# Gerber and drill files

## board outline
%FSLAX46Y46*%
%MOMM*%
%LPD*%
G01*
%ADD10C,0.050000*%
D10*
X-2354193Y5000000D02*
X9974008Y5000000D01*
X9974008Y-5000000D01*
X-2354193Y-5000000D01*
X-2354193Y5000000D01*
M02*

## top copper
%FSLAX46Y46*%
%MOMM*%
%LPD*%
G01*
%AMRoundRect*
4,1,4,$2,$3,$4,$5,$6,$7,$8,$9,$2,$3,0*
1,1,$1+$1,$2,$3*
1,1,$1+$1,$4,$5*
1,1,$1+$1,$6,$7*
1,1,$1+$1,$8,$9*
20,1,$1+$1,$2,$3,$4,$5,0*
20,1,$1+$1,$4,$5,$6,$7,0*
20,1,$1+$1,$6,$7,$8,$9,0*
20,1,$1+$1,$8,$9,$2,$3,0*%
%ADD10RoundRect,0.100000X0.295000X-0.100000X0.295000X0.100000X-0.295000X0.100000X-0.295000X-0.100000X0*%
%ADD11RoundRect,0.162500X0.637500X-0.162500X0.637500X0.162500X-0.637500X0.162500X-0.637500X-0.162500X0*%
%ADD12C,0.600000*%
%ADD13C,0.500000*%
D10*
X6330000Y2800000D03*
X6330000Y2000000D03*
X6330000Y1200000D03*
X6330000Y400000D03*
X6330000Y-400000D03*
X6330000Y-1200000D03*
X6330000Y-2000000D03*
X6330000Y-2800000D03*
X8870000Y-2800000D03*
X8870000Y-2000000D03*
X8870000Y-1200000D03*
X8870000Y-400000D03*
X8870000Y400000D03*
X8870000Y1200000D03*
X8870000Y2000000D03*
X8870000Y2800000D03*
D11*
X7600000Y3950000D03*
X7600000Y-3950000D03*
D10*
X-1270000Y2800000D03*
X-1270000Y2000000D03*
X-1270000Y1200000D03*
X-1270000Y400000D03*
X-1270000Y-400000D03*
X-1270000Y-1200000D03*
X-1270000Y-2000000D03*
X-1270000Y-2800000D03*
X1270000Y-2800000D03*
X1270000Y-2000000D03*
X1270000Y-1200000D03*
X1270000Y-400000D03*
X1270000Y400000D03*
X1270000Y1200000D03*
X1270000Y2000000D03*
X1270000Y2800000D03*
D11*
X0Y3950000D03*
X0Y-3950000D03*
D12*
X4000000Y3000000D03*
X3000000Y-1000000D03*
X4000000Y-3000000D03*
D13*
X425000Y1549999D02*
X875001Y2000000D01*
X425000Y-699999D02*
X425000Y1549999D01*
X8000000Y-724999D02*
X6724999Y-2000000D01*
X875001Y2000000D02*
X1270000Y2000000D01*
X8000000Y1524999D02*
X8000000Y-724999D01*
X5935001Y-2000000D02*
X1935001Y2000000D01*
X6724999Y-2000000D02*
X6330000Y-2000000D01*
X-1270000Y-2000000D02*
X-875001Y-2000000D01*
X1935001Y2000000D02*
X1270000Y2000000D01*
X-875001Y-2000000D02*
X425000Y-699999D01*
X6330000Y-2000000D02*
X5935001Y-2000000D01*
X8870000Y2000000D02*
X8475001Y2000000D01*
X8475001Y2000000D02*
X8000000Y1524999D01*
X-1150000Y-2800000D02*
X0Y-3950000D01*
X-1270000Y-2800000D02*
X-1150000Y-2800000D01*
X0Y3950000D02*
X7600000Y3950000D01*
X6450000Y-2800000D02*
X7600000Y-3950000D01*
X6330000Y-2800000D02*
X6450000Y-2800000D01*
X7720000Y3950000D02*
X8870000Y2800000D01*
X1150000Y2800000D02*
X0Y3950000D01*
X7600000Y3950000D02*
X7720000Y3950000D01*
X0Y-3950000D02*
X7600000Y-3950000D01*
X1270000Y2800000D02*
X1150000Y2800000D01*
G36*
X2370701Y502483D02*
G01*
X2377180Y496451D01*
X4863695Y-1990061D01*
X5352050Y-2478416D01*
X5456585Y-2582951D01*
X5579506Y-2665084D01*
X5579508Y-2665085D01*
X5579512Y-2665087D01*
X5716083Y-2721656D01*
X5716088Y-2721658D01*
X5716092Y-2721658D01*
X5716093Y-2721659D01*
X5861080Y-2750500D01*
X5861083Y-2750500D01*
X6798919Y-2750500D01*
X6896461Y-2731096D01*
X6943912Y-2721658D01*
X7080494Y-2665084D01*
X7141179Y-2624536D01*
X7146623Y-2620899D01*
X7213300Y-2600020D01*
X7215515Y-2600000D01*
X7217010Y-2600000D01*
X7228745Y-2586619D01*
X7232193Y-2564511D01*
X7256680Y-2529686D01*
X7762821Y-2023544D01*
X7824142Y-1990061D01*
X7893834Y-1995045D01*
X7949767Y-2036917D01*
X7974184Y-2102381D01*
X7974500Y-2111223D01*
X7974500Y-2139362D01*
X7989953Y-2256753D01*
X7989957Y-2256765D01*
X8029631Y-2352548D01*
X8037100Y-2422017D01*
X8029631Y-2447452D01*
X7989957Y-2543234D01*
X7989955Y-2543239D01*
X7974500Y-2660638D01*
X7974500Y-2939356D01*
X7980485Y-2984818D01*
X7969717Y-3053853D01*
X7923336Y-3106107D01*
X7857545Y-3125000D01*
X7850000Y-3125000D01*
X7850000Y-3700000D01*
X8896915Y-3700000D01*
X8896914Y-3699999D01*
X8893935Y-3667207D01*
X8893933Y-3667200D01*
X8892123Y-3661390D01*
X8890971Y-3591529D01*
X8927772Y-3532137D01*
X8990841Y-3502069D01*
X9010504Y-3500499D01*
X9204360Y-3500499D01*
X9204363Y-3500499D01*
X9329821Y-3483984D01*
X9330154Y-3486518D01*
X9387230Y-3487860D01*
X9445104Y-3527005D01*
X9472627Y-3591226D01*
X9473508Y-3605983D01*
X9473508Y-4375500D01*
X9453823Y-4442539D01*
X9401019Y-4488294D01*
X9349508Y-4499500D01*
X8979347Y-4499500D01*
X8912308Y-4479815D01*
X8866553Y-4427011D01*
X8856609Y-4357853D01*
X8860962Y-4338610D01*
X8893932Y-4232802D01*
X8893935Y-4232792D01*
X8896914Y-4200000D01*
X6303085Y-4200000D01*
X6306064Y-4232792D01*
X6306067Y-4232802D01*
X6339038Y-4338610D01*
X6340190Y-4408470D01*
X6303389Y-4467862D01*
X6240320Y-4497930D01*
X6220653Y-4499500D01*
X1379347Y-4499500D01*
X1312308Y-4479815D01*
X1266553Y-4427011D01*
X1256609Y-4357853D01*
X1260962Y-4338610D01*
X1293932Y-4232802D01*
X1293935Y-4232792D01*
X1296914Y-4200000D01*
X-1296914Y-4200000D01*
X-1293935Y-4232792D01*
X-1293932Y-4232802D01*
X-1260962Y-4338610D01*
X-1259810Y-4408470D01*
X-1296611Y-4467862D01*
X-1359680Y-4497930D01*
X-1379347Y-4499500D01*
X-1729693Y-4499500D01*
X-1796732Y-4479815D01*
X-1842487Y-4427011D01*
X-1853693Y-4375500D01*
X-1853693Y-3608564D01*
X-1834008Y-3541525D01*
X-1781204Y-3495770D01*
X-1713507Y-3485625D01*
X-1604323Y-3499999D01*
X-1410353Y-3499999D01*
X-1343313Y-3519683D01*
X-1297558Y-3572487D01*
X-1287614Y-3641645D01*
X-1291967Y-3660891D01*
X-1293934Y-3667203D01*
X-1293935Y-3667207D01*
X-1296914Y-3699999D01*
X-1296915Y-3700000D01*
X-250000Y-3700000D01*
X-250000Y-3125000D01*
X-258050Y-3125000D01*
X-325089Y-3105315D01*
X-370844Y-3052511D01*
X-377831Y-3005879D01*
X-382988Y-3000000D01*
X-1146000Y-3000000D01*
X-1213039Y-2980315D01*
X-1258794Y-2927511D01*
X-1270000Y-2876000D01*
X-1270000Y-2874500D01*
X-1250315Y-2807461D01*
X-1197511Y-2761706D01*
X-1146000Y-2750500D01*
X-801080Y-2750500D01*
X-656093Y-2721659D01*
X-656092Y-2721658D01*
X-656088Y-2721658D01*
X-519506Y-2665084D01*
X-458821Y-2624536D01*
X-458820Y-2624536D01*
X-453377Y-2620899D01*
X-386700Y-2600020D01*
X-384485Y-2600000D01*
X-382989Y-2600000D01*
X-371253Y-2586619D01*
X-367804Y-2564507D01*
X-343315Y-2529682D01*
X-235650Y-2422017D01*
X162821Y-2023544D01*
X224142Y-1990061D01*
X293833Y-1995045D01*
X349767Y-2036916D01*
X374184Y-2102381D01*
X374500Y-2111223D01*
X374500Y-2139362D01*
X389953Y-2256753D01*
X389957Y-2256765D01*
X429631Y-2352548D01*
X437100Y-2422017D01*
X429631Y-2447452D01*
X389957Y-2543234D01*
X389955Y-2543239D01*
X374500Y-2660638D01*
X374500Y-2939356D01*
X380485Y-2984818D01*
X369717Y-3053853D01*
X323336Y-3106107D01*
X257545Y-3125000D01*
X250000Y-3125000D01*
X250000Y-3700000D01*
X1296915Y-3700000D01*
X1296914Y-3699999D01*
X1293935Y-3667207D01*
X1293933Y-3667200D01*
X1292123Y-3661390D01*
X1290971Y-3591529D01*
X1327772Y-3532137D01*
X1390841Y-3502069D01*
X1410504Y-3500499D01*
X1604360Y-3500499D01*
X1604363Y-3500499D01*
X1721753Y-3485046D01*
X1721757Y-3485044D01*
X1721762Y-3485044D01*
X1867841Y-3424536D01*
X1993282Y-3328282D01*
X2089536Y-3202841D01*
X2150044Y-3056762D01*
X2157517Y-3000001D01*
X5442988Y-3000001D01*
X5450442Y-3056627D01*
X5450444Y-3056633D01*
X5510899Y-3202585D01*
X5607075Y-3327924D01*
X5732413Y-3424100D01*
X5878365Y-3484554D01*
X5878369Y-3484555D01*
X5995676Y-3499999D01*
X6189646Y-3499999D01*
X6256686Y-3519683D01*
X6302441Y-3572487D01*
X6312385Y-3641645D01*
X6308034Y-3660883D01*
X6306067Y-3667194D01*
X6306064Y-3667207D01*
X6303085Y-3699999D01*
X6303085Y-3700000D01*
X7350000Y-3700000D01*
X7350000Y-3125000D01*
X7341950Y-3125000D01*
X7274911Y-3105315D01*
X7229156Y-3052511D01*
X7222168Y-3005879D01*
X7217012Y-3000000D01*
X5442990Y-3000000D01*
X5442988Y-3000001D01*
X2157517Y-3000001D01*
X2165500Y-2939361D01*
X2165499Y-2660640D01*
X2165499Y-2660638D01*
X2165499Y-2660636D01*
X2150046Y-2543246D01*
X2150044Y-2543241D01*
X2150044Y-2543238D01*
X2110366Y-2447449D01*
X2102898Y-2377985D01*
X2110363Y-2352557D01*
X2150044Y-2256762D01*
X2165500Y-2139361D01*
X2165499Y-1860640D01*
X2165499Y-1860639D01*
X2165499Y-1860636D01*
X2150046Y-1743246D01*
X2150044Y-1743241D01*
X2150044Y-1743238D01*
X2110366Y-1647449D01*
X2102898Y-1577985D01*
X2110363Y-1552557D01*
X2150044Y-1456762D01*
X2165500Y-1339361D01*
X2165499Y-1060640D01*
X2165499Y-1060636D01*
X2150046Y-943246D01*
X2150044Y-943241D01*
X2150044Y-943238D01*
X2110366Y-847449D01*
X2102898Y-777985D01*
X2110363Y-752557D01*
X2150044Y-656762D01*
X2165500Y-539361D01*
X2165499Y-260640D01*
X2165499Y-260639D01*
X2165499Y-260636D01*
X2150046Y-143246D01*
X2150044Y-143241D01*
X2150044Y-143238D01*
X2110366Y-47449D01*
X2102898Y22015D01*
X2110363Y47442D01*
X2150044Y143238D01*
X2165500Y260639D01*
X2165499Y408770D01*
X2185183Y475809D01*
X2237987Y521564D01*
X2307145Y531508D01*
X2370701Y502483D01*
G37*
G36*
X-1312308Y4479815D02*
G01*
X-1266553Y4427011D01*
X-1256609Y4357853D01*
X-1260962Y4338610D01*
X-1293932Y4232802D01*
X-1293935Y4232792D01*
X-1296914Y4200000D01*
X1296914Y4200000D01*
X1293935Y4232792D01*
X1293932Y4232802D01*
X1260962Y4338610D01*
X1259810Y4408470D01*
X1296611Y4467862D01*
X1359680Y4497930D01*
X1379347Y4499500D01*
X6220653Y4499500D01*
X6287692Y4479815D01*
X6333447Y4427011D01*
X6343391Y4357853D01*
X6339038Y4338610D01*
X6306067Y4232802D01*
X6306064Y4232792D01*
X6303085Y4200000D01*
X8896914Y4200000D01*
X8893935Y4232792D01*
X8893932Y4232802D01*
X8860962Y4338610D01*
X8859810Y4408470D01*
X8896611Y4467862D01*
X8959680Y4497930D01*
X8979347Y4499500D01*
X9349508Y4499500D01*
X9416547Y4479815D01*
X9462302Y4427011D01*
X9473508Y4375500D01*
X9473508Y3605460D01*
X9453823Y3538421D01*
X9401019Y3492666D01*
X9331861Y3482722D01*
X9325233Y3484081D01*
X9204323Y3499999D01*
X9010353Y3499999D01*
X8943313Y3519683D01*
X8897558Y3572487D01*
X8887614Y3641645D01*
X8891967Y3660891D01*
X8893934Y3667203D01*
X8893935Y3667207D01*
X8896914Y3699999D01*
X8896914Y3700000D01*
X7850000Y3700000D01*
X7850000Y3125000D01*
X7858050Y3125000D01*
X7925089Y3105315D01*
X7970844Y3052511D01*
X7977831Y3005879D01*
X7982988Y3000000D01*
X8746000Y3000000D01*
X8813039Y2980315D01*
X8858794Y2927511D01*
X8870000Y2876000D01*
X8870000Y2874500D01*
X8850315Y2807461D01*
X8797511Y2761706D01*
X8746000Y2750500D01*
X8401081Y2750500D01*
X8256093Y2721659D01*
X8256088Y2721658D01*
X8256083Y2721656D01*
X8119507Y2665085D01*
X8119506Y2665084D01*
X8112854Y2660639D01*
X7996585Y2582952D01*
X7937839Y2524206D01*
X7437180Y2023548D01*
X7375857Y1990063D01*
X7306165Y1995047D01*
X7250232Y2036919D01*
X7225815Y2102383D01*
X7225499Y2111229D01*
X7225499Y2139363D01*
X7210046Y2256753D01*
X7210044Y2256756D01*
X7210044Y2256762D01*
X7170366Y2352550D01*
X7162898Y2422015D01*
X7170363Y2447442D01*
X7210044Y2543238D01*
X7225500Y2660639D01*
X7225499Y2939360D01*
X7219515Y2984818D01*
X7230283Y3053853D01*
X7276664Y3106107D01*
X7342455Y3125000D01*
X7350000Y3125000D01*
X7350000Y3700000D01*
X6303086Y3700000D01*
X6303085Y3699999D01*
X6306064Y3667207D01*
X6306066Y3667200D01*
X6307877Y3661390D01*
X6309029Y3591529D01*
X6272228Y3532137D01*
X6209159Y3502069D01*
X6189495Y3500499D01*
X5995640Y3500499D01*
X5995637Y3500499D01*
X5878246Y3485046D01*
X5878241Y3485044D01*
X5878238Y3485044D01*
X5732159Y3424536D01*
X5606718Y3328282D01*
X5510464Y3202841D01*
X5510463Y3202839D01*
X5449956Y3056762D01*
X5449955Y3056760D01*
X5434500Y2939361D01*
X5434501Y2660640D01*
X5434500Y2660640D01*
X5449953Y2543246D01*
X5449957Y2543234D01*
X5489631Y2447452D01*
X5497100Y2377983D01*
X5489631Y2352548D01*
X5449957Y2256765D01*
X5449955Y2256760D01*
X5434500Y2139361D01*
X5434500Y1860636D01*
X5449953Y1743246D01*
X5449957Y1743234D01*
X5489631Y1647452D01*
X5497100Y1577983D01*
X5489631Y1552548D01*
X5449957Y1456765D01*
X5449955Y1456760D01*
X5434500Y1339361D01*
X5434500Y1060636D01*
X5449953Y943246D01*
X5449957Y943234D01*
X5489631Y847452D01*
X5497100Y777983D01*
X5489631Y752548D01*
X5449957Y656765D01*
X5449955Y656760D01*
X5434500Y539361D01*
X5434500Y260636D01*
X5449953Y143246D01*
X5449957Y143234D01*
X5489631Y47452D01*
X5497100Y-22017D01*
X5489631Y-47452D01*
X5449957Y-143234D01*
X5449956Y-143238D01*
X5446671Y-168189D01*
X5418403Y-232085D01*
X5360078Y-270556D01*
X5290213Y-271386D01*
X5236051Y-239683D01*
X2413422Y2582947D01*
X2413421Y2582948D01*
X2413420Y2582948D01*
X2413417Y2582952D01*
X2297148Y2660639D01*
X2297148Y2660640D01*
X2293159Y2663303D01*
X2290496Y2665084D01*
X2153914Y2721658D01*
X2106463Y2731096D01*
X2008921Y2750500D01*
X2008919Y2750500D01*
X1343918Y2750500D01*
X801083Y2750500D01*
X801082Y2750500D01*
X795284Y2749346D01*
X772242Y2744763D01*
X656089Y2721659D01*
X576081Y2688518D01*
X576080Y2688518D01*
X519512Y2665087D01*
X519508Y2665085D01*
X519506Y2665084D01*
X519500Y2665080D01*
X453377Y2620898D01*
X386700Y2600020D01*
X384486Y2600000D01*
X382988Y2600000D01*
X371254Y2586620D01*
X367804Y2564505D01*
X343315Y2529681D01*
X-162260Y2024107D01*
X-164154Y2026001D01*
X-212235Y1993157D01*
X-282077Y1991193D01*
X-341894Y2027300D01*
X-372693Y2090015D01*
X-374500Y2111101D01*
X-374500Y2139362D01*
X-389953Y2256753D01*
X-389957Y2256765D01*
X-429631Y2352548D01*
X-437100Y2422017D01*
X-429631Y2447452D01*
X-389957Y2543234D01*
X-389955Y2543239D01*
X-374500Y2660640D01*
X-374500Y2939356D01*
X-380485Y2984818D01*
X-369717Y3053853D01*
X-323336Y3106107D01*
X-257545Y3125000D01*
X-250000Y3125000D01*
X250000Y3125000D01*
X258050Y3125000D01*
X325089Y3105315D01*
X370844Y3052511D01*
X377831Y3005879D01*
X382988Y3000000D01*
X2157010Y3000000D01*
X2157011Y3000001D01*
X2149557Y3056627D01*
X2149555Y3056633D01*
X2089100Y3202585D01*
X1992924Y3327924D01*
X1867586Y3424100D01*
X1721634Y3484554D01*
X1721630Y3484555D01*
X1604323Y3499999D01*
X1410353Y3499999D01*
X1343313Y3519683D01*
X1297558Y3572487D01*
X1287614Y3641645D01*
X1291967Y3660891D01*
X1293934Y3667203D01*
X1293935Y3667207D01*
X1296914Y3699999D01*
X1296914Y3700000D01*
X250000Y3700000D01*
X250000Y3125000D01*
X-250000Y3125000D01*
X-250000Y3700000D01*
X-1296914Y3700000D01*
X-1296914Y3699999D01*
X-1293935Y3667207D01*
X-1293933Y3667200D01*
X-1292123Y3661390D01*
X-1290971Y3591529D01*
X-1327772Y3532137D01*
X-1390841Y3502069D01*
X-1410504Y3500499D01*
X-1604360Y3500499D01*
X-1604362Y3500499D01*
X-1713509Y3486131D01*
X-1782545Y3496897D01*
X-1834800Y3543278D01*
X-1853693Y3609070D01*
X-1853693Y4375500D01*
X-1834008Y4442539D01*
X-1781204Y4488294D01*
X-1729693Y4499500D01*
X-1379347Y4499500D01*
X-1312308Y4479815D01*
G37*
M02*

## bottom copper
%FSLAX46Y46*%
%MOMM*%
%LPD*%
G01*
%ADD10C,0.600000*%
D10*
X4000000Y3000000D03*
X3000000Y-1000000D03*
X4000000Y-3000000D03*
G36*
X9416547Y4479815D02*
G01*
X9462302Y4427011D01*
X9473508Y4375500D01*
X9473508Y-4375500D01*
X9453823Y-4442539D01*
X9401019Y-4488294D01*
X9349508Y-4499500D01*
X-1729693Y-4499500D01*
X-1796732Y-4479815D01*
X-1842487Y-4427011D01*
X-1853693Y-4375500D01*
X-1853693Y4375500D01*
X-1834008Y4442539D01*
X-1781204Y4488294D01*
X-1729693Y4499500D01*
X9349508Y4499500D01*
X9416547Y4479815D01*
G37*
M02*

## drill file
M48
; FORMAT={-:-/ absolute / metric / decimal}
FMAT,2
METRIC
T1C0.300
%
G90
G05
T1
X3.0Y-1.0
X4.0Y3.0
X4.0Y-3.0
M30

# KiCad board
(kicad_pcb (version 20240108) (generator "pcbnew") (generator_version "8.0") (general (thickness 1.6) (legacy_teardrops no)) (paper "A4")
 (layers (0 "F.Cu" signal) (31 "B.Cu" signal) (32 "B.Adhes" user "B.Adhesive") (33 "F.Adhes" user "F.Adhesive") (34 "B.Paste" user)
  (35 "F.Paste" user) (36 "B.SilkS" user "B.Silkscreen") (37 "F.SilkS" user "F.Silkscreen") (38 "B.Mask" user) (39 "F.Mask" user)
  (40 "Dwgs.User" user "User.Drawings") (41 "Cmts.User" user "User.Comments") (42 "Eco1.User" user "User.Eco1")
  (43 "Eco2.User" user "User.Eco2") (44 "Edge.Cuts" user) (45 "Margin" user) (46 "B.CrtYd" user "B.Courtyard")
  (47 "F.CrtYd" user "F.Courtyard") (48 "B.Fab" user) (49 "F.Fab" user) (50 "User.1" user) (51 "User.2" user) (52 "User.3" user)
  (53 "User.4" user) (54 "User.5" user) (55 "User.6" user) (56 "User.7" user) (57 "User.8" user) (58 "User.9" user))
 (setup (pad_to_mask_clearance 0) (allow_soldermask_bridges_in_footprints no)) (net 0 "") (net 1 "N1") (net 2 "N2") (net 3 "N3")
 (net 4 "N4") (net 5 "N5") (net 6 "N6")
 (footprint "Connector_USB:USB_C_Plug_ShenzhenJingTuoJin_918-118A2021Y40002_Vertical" (layer "F.Cu") (at 7.6 0)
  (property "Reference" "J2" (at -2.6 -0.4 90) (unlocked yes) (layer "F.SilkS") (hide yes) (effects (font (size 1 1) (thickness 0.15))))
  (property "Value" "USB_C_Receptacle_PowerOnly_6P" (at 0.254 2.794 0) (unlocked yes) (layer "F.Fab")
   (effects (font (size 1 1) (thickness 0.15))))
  (pad "A1" smd roundrect (at -1.27 -2.8 90) (size 0.4 0.79) (layers "F.Cu" "F.Paste" "F.Mask") (roundrect_rratio 0.25))
  (pad "A4" smd roundrect (at -1.27 -2 90) (size 0.4 0.79) (layers "F.Cu" "F.Paste" "F.Mask") (roundrect_rratio 0.25))
  (pad "A5" smd roundrect (at -1.27 -1.2 90) (size 0.4 0.79) (layers "F.Cu" "F.Paste" "F.Mask") (roundrect_rratio 0.25) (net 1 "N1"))
  (pad "A6" smd roundrect (at -1.27 -0.4 90) (size 0.4 0.79) (layers "F.Cu" "F.Paste" "F.Mask") (roundrect_rratio 0.25))
  (pad "A7" smd roundrect (at -1.27 0.4 90) (size 0.4 0.79) (layers "F.Cu" "F.Paste" "F.Mask") (roundrect_rratio 0.25))
  (pad "A8" smd roundrect (at -1.27 1.2 90) (size 0.4 0.79) (layers "F.Cu" "F.Paste" "F.Mask") (roundrect_rratio 0.25))
  (pad "A9" smd roundrect (at -1.27 2 90) (size 0.4 0.79) (layers "F.Cu" "F.Paste" "F.Mask") (roundrect_rratio 0.25) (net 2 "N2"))
  (pad "A12" smd roundrect (at -1.27 2.8 90) (size 0.4 0.79) (layers "F.Cu" "F.Paste" "F.Mask") (roundrect_rratio 0.25) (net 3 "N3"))
  (pad "B1" smd roundrect (at 1.27 2.8 90) (size 0.4 0.79) (layers "F.Cu" "F.Paste" "F.Mask") (roundrect_rratio 0.25))
  (pad "B4" smd roundrect (at 1.27 2 90) (size 0.4 0.79) (layers "F.Cu" "F.Paste" "F.Mask") (roundrect_rratio 0.25))
  (pad "B5" smd roundrect (at 1.27 1.2 90) (size 0.4 0.79) (layers "F.Cu" "F.Paste" "F.Mask") (roundrect_rratio 0.25) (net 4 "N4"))
  (pad "B6" smd roundrect (at 1.27 0.4 90) (size 0.4 0.79) (layers "F.Cu" "F.Paste" "F.Mask") (roundrect_rratio 0.25))
  (pad "B7" smd roundrect (at 1.27 -0.4 90) (size 0.4 0.79) (layers "F.Cu" "F.Paste" "F.Mask") (roundrect_rratio 0.25))
  (pad "B8" smd roundrect (at 1.27 -1.2 90) (size 0.4 0.79) (layers "F.Cu" "F.Paste" "F.Mask") (roundrect_rratio 0.25))
  (pad "B9" smd roundrect (at 1.27 -2 90) (size 0.4 0.79) (layers "F.Cu" "F.Paste" "F.Mask") (roundrect_rratio 0.25) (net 2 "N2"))
  (pad "B12" smd roundrect (at 1.27 -2.8 90) (size 0.4 0.79) (layers "F.Cu" "F.Paste" "F.Mask") (roundrect_rratio 0.25) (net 3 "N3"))
  (pad "S1" smd roundrect (at 0 -3.95 90) (size 0.65 1.6) (layers "F.Cu" "F.Paste" "F.Mask") (roundrect_rratio 0.25) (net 3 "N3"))
  (pad "S1" smd roundrect (at 0 3.95 90) (size 0.65 1.6) (layers "F.Cu" "F.Paste" "F.Mask") (roundrect_rratio 0.25) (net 3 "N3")))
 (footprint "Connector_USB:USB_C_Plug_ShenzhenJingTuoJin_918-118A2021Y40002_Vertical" (layer "F.Cu") (at 0 0)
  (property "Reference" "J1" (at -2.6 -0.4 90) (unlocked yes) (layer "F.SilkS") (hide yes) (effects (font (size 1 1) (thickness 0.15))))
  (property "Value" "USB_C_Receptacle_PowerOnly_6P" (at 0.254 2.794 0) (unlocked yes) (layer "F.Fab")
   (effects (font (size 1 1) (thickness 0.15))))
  (pad "A1" smd roundrect (at -1.27 -2.8 90) (size 0.4 0.79) (layers "F.Cu" "F.Paste" "F.Mask") (roundrect_rratio 0.25))
  (pad "A4" smd roundrect (at -1.27 -2 90) (size 0.4 0.79) (layers "F.Cu" "F.Paste" "F.Mask") (roundrect_rratio 0.25))
  (pad "A5" smd roundrect (at -1.27 -1.2 90) (size 0.4 0.79) (layers "F.Cu" "F.Paste" "F.Mask") (roundrect_rratio 0.25) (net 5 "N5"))
  (pad "A6" smd roundrect (at -1.27 -0.4 90) (size 0.4 0.79) (layers "F.Cu" "F.Paste" "F.Mask") (roundrect_rratio 0.25))
  (pad "A7" smd roundrect (at -1.27 0.4 90) (size 0.4 0.79) (layers "F.Cu" "F.Paste" "F.Mask") (roundrect_rratio 0.25))
  (pad "A8" smd roundrect (at -1.27 1.2 90) (size 0.4 0.79) (layers "F.Cu" "F.Paste" "F.Mask") (roundrect_rratio 0.25))
  (pad "A9" smd roundrect (at -1.27 2 90) (size 0.4 0.79) (layers "F.Cu" "F.Paste" "F.Mask") (roundrect_rratio 0.25) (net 2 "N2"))
  (pad "A12" smd roundrect (at -1.27 2.8 90) (size 0.4 0.79) (layers "F.Cu" "F.Paste" "F.Mask") (roundrect_rratio 0.25) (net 3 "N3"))
  (pad "B1" smd roundrect (at 1.27 2.8 90) (size 0.4 0.79) (layers "F.Cu" "F.Paste" "F.Mask") (roundrect_rratio 0.25))
  (pad "B4" smd roundrect (at 1.27 2 90) (size 0.4 0.79) (layers "F.Cu" "F.Paste" "F.Mask") (roundrect_rratio 0.25))
  (pad "B5" smd roundrect (at 1.27 1.2 90) (size 0.4 0.79) (layers "F.Cu" "F.Paste" "F.Mask") (roundrect_rratio 0.25) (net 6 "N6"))
  (pad "B6" smd roundrect (at 1.27 0.4 90) (size 0.4 0.79) (layers "F.Cu" "F.Paste" "F.Mask") (roundrect_rratio 0.25))
  (pad "B7" smd roundrect (at 1.27 -0.4 90) (size 0.4 0.79) (layers "F.Cu" "F.Paste" "F.Mask") (roundrect_rratio 0.25))
  (pad "B8" smd roundrect (at 1.27 -1.2 90) (size 0.4 0.79) (layers "F.Cu" "F.Paste" "F.Mask") (roundrect_rratio 0.25))
  (pad "B9" smd roundrect (at 1.27 -2 90) (size 0.4 0.79) (layers "F.Cu" "F.Paste" "F.Mask") (roundrect_rratio 0.25) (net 2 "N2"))
  (pad "B12" smd roundrect (at 1.27 -2.8 90) (size 0.4 0.79) (layers "F.Cu" "F.Paste" "F.Mask") (roundrect_rratio 0.25) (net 3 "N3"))
  (pad "S1" smd roundrect (at 0 -3.95 90) (size 0.65 1.6) (layers "F.Cu" "F.Paste" "F.Mask") (roundrect_rratio 0.25) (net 3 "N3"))
  (pad "S1" smd roundrect (at 0 3.95 90) (size 0.65 1.6) (layers "F.Cu" "F.Paste" "F.Mask") (roundrect_rratio 0.25) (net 3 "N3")))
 (gr_rect (start -2.354193 -5) (end 9.974008 5) (stroke (width 0.05) (type default)) (fill none) (layer "Edge.Cuts"))
 (segment (start 0.425 -1.549999) (end 0.875001 -2) (width 0.5) (layer "F.Cu") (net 2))
 (segment (start 0.425 0.699999) (end 0.425 -1.549999) (width 0.5) (layer "F.Cu") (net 2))
 (segment (start 8 0.724999) (end 6.724999 2) (width 0.5) (layer "F.Cu") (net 2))
 (segment (start 0.875001 -2) (end 1.27 -2) (width 0.5) (layer "F.Cu") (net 2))
 (segment (start 8 -1.524999) (end 8 0.724999) (width 0.5) (layer "F.Cu") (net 2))
 (segment (start 5.935001 2) (end 1.935001 -2) (width 0.5) (layer "F.Cu") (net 2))
 (segment (start 6.724999 2) (end 6.33 2) (width 0.5) (layer "F.Cu") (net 2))
 (segment (start -1.27 2) (end -0.875001 2) (width 0.5) (layer "F.Cu") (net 2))
 (segment (start 1.935001 -2) (end 1.27 -2) (width 0.5) (layer "F.Cu") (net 2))
 (segment (start -0.875001 2) (end 0.425 0.699999) (width 0.5) (layer "F.Cu") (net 2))
 (segment (start 6.33 2) (end 5.935001 2) (width 0.5) (layer "F.Cu") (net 2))
 (segment (start 8.87 -2) (end 8.475001 -2) (width 0.5) (layer "F.Cu") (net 2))
 (segment (start 8.475001 -2) (end 8 -1.524999) (width 0.5) (layer "F.Cu") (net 2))
 (segment (start -1.15 2.8) (end 0 3.95) (width 0.5) (layer "F.Cu") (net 3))
 (segment (start -1.27 2.8) (end -1.15 2.8) (width 0.5) (layer "F.Cu") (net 3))
 (segment (start 0 -3.95) (end 7.6 -3.95) (width 0.5) (layer "F.Cu") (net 3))
 (segment (start 6.45 2.8) (end 7.6 3.95) (width 0.5) (layer "F.Cu") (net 3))
 (segment (start 6.33 2.8) (end 6.45 2.8) (width 0.5) (layer "F.Cu") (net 3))
 (segment (start 7.72 -3.95) (end 8.87 -2.8) (width 0.5) (layer "F.Cu") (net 3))
 (segment (start 1.15 -2.8) (end 0 -3.95) (width 0.5) (layer "F.Cu") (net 3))
 (segment (start 7.6 -3.95) (end 7.72 -3.95) (width 0.5) (layer "F.Cu") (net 3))
 (segment (start 0 3.95) (end 7.6 3.95) (width 0.5) (layer "F.Cu") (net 3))
 (segment (start 1.27 -2.8) (end 1.15 -2.8) (width 0.5) (layer "F.Cu") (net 3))
 (via (at 4 -3) (size 0.6) (drill 0.3) (layers "F.Cu" "B.Cu") (free yes) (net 3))
 (via (at 3 1) (size 0.6) (drill 0.3) (layers "F.Cu" "B.Cu") (free yes) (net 3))
 (via (at 4 3) (size 0.6) (drill 0.3) (layers "F.Cu" "B.Cu") (free yes) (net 3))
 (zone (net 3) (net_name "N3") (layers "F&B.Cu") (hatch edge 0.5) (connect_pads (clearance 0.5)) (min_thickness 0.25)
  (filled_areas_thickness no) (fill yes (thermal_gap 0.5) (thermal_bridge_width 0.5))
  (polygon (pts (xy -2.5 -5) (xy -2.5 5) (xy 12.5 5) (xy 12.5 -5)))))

